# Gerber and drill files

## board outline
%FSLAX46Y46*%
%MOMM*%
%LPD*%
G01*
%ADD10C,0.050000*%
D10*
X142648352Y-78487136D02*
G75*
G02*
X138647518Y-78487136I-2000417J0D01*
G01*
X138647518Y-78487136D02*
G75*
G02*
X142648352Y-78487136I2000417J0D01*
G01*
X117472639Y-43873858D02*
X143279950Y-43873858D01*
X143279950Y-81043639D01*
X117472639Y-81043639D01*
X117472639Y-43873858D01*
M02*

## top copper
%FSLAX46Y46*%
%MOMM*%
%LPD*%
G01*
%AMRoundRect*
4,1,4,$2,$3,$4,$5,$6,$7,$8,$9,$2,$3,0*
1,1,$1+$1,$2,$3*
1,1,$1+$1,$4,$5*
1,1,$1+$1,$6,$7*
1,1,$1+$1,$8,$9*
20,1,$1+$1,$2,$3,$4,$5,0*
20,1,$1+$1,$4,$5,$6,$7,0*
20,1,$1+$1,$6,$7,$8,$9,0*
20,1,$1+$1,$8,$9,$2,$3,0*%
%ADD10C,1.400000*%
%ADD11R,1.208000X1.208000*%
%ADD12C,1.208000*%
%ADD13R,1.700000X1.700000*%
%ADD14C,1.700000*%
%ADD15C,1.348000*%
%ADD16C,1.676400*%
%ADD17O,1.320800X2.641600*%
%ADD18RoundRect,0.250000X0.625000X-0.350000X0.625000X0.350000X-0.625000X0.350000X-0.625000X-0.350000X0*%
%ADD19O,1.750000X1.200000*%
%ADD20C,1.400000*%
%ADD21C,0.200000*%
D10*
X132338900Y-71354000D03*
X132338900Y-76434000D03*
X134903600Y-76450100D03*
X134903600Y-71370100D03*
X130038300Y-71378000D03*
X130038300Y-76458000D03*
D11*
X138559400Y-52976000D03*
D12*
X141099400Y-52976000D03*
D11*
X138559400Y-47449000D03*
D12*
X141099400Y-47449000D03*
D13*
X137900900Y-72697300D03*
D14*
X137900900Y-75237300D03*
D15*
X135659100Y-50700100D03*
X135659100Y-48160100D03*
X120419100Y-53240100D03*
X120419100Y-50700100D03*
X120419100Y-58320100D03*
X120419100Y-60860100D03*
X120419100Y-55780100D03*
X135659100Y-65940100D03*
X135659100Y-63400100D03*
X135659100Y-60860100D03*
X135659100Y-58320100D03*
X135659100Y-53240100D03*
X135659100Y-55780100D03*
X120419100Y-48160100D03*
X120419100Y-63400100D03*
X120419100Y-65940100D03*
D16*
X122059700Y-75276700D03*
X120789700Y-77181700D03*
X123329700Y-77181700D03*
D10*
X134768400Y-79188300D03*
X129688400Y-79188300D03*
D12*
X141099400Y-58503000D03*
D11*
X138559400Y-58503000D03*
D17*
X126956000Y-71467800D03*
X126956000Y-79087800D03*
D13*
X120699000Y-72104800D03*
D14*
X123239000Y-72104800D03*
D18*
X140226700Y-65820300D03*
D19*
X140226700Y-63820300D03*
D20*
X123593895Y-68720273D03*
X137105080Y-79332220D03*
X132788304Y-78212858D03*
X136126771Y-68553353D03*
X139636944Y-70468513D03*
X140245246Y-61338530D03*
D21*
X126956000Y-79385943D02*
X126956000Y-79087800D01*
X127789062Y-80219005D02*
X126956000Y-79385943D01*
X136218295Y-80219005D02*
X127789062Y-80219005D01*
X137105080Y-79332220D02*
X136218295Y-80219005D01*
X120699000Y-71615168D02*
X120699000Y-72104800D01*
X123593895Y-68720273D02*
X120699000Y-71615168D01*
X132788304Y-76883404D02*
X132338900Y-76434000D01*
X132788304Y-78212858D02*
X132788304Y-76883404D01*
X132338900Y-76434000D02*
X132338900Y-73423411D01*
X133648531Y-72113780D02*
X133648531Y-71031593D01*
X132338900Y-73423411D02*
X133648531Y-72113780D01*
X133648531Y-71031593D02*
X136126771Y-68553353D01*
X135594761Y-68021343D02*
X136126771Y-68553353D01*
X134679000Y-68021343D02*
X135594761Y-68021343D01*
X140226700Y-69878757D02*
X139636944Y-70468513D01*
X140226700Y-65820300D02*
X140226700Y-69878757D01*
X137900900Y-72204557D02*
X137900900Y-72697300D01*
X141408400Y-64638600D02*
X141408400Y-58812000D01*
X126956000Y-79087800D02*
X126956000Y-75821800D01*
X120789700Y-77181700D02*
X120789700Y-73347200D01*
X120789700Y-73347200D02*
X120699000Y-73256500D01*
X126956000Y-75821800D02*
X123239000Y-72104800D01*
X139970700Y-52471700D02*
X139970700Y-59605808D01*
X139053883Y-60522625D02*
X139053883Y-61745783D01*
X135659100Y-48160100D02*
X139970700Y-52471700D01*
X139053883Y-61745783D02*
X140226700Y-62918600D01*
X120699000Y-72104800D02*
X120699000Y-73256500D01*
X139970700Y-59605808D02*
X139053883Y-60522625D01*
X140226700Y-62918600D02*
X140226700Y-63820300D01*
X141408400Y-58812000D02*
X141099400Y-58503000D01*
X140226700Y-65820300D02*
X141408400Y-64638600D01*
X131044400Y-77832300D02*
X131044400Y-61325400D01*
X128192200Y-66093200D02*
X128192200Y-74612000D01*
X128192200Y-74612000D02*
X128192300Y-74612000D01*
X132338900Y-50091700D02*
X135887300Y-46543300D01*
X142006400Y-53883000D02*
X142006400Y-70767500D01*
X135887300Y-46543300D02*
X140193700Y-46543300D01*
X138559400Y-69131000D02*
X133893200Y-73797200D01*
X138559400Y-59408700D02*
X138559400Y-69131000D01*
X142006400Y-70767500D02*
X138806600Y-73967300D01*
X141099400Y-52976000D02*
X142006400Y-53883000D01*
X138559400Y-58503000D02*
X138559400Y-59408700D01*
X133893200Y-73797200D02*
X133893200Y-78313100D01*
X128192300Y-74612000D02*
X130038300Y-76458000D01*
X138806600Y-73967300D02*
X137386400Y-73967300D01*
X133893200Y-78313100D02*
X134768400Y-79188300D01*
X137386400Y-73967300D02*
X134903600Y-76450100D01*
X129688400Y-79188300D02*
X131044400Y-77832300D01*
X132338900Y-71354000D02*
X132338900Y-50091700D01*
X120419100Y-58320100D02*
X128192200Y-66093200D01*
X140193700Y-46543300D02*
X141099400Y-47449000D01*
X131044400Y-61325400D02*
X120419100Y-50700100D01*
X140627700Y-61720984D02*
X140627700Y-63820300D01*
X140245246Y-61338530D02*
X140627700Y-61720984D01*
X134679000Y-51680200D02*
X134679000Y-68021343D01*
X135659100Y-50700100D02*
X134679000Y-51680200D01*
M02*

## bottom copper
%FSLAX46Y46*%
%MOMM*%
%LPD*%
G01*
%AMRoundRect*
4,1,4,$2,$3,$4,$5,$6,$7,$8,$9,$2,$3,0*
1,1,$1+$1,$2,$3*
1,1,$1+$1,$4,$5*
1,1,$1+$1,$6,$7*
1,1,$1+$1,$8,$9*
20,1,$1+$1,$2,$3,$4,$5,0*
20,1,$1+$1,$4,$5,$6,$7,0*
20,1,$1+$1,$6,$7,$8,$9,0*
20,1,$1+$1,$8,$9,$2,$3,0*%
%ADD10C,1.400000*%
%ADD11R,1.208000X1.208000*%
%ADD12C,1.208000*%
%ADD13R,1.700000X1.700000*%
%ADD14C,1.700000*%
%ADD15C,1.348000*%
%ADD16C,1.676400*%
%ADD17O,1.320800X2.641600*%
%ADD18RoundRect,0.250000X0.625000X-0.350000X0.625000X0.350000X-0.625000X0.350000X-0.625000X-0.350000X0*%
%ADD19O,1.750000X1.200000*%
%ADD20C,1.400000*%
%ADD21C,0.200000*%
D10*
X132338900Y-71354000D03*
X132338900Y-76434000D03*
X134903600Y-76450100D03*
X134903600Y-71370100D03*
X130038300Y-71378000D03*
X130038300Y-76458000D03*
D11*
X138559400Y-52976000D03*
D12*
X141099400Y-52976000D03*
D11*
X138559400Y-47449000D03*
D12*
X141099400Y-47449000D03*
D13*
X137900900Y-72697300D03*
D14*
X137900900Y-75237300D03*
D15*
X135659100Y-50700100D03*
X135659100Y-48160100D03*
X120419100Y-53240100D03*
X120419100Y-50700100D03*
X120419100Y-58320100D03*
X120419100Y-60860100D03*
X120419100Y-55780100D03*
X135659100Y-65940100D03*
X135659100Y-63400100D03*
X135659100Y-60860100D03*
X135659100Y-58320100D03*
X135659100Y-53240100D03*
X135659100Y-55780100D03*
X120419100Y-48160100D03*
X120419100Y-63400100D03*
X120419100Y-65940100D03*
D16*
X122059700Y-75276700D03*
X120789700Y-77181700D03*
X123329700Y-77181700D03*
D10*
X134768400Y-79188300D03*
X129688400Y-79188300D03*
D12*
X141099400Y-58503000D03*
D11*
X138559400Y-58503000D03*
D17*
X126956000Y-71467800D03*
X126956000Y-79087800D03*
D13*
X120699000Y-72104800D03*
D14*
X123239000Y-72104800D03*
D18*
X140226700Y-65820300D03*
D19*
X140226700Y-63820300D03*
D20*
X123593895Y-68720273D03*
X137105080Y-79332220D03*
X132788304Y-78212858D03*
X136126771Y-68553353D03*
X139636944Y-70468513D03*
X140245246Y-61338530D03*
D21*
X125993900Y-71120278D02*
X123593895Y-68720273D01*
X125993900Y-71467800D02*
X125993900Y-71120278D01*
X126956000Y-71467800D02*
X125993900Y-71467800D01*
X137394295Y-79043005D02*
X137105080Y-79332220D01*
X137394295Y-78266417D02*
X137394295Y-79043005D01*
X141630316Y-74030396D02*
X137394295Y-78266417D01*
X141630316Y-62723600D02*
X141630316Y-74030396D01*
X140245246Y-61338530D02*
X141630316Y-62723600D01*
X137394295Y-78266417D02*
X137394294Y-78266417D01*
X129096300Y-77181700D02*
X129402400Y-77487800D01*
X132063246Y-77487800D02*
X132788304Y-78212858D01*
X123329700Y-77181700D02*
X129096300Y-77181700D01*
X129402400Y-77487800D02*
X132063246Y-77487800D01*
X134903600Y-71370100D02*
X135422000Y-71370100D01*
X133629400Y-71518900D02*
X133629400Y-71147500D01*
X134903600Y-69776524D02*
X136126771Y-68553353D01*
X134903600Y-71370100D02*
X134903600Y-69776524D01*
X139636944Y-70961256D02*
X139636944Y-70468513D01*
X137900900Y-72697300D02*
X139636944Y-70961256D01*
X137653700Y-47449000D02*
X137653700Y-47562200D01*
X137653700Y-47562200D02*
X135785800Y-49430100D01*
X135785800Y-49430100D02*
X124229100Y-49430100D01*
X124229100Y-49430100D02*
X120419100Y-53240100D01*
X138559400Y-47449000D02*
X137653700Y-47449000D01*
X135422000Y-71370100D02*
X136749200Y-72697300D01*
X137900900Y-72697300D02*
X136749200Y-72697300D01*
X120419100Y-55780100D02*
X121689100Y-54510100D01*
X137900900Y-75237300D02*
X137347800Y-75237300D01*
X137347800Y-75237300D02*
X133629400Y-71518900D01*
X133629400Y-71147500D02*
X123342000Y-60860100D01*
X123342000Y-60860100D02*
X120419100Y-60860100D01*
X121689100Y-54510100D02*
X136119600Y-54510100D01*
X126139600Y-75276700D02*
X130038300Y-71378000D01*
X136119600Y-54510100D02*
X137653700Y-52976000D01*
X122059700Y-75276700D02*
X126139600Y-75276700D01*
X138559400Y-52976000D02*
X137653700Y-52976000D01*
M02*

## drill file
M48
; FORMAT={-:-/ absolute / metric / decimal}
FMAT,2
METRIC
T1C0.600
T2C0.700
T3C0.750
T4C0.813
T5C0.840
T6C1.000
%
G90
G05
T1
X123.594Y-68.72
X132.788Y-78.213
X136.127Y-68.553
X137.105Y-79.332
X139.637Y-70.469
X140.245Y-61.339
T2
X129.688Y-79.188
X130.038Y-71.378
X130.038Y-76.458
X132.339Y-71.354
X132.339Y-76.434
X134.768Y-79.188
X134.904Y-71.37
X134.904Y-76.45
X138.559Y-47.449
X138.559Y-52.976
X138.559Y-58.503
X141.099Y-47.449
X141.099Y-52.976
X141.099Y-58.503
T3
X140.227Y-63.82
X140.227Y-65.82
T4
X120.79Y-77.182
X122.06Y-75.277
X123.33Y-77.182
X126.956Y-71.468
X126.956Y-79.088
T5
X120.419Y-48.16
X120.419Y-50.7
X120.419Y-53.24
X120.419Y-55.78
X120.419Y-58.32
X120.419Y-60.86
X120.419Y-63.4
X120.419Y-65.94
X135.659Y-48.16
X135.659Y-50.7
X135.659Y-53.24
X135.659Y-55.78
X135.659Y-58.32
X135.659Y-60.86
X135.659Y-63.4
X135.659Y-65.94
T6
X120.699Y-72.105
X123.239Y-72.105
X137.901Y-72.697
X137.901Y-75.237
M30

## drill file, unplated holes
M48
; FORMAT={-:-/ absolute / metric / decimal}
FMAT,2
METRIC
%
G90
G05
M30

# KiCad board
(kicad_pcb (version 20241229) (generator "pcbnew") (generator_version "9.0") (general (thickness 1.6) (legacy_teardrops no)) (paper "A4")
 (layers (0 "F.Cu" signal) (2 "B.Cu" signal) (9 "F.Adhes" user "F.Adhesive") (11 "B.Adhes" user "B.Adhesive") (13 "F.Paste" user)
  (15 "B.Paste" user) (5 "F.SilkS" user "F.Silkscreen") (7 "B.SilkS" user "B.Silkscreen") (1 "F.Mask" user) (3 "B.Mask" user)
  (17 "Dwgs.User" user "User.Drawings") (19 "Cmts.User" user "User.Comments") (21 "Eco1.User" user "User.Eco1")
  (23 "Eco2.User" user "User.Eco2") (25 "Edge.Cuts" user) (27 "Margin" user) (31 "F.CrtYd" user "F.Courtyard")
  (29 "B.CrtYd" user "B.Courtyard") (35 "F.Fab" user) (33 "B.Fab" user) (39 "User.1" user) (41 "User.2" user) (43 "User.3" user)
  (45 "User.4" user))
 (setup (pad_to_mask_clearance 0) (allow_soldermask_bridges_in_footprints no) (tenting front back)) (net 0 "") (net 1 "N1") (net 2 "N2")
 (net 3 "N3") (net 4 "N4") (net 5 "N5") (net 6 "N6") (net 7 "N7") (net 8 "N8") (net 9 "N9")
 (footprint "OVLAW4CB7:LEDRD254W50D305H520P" (layer "F.Cu") (at 139.8294 52.976)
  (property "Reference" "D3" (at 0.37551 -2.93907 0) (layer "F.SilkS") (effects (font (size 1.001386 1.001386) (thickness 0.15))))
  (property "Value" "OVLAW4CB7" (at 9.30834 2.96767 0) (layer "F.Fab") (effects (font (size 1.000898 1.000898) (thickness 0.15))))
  (pad "A" thru_hole rect (at -1.27 0) (size 1.208 1.208) (drill 0.7) (layers "*.Cu" "*.Mask") (remove_unused_layers no)
   (solder_mask_margin 0.102))
  (pad "C" thru_hole circle (at 1.27 0) (size 1.208 1.208) (drill 0.7) (layers "*.Cu" "*.Mask") (remove_unused_layers no)
   (solder_mask_margin 0.102)))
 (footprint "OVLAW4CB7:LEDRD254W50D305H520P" (layer "F.Cu") (at 139.8294 47.449)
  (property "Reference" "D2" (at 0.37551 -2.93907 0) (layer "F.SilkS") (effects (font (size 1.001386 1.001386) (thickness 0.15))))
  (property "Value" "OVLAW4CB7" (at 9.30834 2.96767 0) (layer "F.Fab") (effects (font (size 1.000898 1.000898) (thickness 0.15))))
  (pad "A" thru_hole rect (at -1.27 0) (size 1.208 1.208) (drill 0.7) (layers "*.Cu" "*.Mask") (remove_unused_layers no)
   (solder_mask_margin 0.102))
  (pad "C" thru_hole circle (at 1.27 0) (size 1.208 1.208) (drill 0.7) (layers "*.Cu" "*.Mask") (remove_unused_layers no)
   (solder_mask_margin 0.102)))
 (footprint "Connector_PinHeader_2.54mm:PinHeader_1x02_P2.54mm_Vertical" (layer "F.Cu") (at 137.9009 72.6973)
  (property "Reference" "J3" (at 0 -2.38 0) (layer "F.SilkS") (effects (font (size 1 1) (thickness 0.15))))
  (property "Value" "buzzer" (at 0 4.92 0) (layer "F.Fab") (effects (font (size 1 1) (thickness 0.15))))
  (pad "1" thru_hole rect (at 0 0) (size 1.7 1.7) (drill 1) (layers "*.Cu" "*.Mask") (remove_unused_layers no))
  (pad "2" thru_hole circle (at 0 2.54) (size 1.7 1.7) (drill 1) (layers "*.Cu" "*.Mask") (remove_unused_layers no)))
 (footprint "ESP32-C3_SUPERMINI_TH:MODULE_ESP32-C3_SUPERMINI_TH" (layer "F.Cu") (at 128.0391 58.0601)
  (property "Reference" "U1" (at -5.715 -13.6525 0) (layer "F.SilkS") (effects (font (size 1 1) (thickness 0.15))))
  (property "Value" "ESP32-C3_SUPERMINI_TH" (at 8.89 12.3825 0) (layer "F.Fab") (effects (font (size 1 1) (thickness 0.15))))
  (pad "0" thru_hole circle (at 7.62 7.88) (size 1.348 1.348) (drill 0.84) (layers "*.Cu" "*.Mask") (remove_unused_layers no) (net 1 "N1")
   (solder_mask_margin 0.102))
  (pad "1" thru_hole circle (at 7.62 5.34) (size 1.348 1.348) (drill 0.84) (layers "*.Cu" "*.Mask") (remove_unused_layers no) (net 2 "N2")
   (solder_mask_margin 0.102))
  (pad "2" thru_hole circle (at 7.62 2.8) (size 1.348 1.348) (drill 0.84) (layers "*.Cu" "*.Mask") (remove_unused_layers no) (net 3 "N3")
   (solder_mask_margin 0.102))
  (pad "3" thru_hole circle (at 7.62 0.26) (size 1.348 1.348) (drill 0.84) (layers "*.Cu" "*.Mask") (remove_unused_layers no) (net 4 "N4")
   (solder_mask_margin 0.102))
  (pad "3.3" thru_hole circle (at 7.62 -4.82) (size 1.348 1.348) (drill 0.84) (layers "*.Cu" "*.Mask") (remove_unused_layers no)
   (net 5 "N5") (solder_mask_margin 0.102))
  (pad "4" thru_hole circle (at 7.62 -2.28) (size 1.348 1.348) (drill 0.84) (layers "*.Cu" "*.Mask") (remove_unused_layers no) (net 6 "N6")
   (solder_mask_margin 0.102))
  (pad "5" thru_hole circle (at -7.62 -9.9) (size 1.348 1.348) (drill 0.84) (layers "*.Cu" "*.Mask") (remove_unused_layers no) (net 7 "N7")
   (solder_mask_margin 0.102))
  (pad "5V" thru_hole circle (at 7.62 -9.9) (size 1.348 1.348) (drill 0.84) (layers "*.Cu" "*.Mask") (remove_unused_layers no)
   (solder_mask_margin 0.102))
  (pad "6" thru_hole circle (at -7.62 -7.36) (size 1.348 1.348) (drill 0.84) (layers "*.Cu" "*.Mask") (remove_unused_layers no)
   (solder_mask_margin 0.102))
  (pad "7" thru_hole circle (at -7.62 -4.82) (size 1.348 1.348) (drill 0.84) (layers "*.Cu" "*.Mask") (remove_unused_layers no)
   (solder_mask_margin 0.102))
  (pad "8" thru_hole circle (at -7.62 -2.28) (size 1.348 1.348) (drill 0.84) (layers "*.Cu" "*.Mask") (remove_unused_layers no)
   (solder_mask_margin 0.102))
  (pad "9" thru_hole circle (at -7.62 0.26) (size 1.348 1.348) (drill 0.84) (layers "*.Cu" "*.Mask") (remove_unused_layers no)
   (solder_mask_margin 0.102))
  (pad "10" thru_hole circle (at -7.62 2.8) (size 1.348 1.348) (drill 0.84) (layers "*.Cu" "*.Mask") (remove_unused_layers no)
   (solder_mask_margin 0.102))
  (pad "20" thru_hole circle (at -7.62 5.34) (size 1.348 1.348) (drill 0.84) (layers "*.Cu" "*.Mask") (remove_unused_layers no) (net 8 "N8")
   (solder_mask_margin 0.102))
  (pad "21" thru_hole circle (at -7.62 7.88) (size 1.348 1.348) (drill 0.84) (layers "*.Cu" "*.Mask") (remove_unused_layers no) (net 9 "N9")
   (solder_mask_margin 0.102))
  (pad "G" thru_hole circle (at 7.62 -7.36) (size 1.348 1.348) (drill 0.84) (layers "*.Cu" "*.Mask") (remove_unused_layers no)
   (solder_mask_margin 0.102)))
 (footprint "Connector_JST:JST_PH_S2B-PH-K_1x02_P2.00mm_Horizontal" (layer "F.Cu") (at 140.2267 65.8203 90)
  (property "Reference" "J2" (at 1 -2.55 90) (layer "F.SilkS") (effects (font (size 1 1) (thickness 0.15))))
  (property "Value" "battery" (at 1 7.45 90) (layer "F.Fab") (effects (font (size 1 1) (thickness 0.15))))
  (pad "1" thru_hole roundrect (at 0 0 90) (size 1.2 1.75) (drill 0.75) (layers "*.Cu" "*.Mask") (remove_unused_layers no)
   (roundrect_rratio 0.208333))
  (pad "2" thru_hole oval (at 2 0 90) (size 1.2 1.75) (drill 0.75) (layers "*.Cu" "*.Mask") (remove_unused_layers no)))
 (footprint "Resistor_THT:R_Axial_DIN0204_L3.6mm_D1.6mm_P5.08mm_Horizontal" (layer "F.Cu") (at 134.9036 76.4501 90)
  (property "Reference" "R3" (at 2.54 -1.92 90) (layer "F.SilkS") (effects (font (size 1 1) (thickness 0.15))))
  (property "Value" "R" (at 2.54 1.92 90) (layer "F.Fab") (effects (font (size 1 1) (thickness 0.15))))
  (pad "1" thru_hole circle (at 0 0 90) (size 1.4 1.4) (drill 0.7) (layers "*.Cu" "*.Mask") (remove_unused_layers no))
  (pad "2" thru_hole circle (at 5.08 0 90) (size 1.4 1.4) (drill 0.7) (layers "*.Cu" "*.Mask") (remove_unused_layers no)))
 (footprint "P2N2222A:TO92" (layer "F.Cu") (at 122.0597 77.1817)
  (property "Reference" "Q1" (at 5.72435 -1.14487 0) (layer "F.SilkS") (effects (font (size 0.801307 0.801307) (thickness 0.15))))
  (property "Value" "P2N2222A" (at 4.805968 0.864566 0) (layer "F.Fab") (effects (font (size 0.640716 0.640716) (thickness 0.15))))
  (pad "1" thru_hole circle (at 1.27 0) (size 1.6764 1.6764) (drill 0.8128) (layers "*.Cu" "*.Mask") (remove_unused_layers no)
   (solder_mask_margin 0.102))
  (pad "2" thru_hole circle (at 0 -1.905) (size 1.6764 1.6764) (drill 0.8128) (layers "*.Cu" "*.Mask") (remove_unused_layers no)
   (solder_mask_margin 0.102))
  (pad "3" thru_hole circle (at -1.27 0) (size 1.6764 1.6764) (drill 0.8128) (layers "*.Cu" "*.Mask") (remove_unused_layers no)
   (solder_mask_margin 0.102)))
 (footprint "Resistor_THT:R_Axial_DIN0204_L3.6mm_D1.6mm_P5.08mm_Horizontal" (layer "F.Cu") (at 130.0383 76.458 90)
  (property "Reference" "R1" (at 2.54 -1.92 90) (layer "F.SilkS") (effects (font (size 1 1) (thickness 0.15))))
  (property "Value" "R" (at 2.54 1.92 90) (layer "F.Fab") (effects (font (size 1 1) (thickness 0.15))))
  (pad "1" thru_hole circle (at 0 0 90) (size 1.4 1.4) (drill 0.7) (layers "*.Cu" "*.Mask") (remove_unused_layers no))
  (pad "2" thru_hole circle (at 5.08 0 90) (size 1.4 1.4) (drill 0.7) (layers "*.Cu" "*.Mask") (remove_unused_layers no)))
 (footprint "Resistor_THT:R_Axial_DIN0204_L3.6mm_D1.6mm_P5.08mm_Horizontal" (layer "F.Cu") (at 132.3389 71.354 -90)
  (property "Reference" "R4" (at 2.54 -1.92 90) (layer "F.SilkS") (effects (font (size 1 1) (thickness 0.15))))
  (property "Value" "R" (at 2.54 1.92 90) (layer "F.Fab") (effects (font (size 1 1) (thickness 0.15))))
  (pad "1" thru_hole circle (at 0 0 270) (size 1.4 1.4) (drill 0.7) (layers "*.Cu" "*.Mask") (remove_unused_layers no))
  (pad "2" thru_hole circle (at 5.08 0 270) (size 1.4 1.4) (drill 0.7) (layers "*.Cu" "*.Mask") (remove_unused_layers no)))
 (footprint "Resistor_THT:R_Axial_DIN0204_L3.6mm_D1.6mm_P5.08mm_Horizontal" (layer "F.Cu") (at 134.7684 79.1883 180)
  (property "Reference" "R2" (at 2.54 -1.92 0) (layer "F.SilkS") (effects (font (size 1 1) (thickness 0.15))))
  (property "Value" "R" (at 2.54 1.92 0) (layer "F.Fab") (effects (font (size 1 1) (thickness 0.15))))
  (pad "1" thru_hole circle (at 0 0 180) (size 1.4 1.4) (drill 0.7) (layers "*.Cu" "*.Mask") (remove_unused_layers no))
  (pad "2" thru_hole circle (at 5.08 0 180) (size 1.4 1.4) (drill 0.7) (layers "*.Cu" "*.Mask") (remove_unused_layers no)))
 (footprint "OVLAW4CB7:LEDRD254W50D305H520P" (layer "F.Cu") (at 139.8294 58.503)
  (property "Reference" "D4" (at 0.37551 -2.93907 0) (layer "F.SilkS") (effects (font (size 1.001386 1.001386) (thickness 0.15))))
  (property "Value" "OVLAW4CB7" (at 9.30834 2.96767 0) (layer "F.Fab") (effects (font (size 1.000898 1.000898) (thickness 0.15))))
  (pad "A" thru_hole rect (at -1.27 0) (size 1.208 1.208) (drill 0.7) (layers "*.Cu" "*.Mask") (remove_unused_layers no)
   (solder_mask_margin 0.102))
  (pad "C" thru_hole circle (at 1.27 0) (size 1.208 1.208) (drill 0.7) (layers "*.Cu" "*.Mask") (remove_unused_layers no)
   (solder_mask_margin 0.102)))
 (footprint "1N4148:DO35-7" (layer "F.Cu") (at 126.956 75.2778 90)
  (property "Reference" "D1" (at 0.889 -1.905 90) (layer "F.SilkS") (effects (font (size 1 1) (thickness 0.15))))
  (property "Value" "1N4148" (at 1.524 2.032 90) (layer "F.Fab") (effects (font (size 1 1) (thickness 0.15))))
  (pad "A" thru_hole oval (at 3.81 0 90) (size 2.6416 1.3208) (drill 0.8128) (layers "*.Cu" "*.Mask") (remove_unused_layers no)
   (solder_mask_margin 0.102))
  (pad "C" thru_hole oval (at -3.81 0 90) (size 2.6416 1.3208) (drill 0.8128) (layers "*.Cu" "*.Mask") (remove_unused_layers no)
   (solder_mask_margin 0.102)))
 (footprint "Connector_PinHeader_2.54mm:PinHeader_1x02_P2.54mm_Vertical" (layer "F.Cu") (at 120.699 72.1048 90)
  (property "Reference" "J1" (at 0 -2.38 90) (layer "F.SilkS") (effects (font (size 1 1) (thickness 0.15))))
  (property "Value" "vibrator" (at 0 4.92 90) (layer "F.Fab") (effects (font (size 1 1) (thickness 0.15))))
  (pad "1" thru_hole rect (at 0 0 90) (size 1.7 1.7) (drill 1) (layers "*.Cu" "*.Mask") (remove_unused_layers no))
  (pad "2" thru_hole circle (at 0 2.54 90) (size 1.7 1.7) (drill 1) (layers "*.Cu" "*.Mask") (remove_unused_layers no)))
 (gr_circle (center 140.647935 78.487136) (end 138.891232 79.444039) (stroke (width 0.05) (type default)) (fill no) (layer "Edge.Cuts"))
 (gr_rect (start 117.472639 43.873858) (end 143.27995 81.043639) (stroke (width 0.05) (type default)) (fill no) (layer "Edge.Cuts"))
 (segment (start 127.789062 80.219005) (end 126.956 79.385943) (width 0.2) (layer "F.Cu") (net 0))
 (segment (start 132.788304 78.212858) (end 132.788304 76.883404) (width 0.2) (layer "F.Cu") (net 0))
 (segment (start 137.3864 73.9673) (end 134.9036 76.4501) (width 0.2) (layer "F.Cu") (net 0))
 (segment (start 140.1937 46.5433) (end 141.0994 47.449) (width 0.2) (layer "F.Cu") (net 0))
 (segment (start 128.1923 74.612) (end 130.0383 76.458) (width 0.2) (layer "F.Cu") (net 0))
 (segment (start 138.8066 73.9673) (end 137.3864 73.9673) (width 0.2) (layer "F.Cu") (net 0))
 (segment (start 134.679 51.6802) (end 134.679 68.021343) (width 0.2) (layer "F.Cu") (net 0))
 (segment (start 140.2267 65.8203) (end 140.2267 69.878757) (width 0.2) (layer "F.Cu") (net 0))
 (segment (start 120.7897 77.1817) (end 120.7897 73.3472) (width 0.2) (layer "F.Cu") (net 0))
 (segment (start 139.9707 52.4717) (end 139.9707 59.605808) (width 0.2) (layer "F.Cu") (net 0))
 (segment (start 136.218295 80.219005) (end 127.789062 80.219005) (width 0.2) (layer "F.Cu") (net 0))
 (segment (start 141.4084 58.812) (end 141.0994 58.503) (width 0.2) (layer "F.Cu") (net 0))
 (segment (start 132.3389 71.354) (end 132.3389 50.0917) (width 0.2) (layer "F.Cu") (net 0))
 (segment (start 142.0064 70.7675) (end 138.8066 73.9673) (width 0.2) (layer "F.Cu") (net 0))
 (segment (start 132.3389 50.0917) (end 135.8873 46.5433) (width 0.2) (layer "F.Cu") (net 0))
 (segment (start 133.648531 72.11378) (end 133.648531 71.031593) (width 0.2) (layer "F.Cu") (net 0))
 (segment (start 120.699 72.1048) (end 120.699 73.2565) (width 0.2) (layer "F.Cu") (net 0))
 (segment (start 135.594761 68.021343) (end 136.126771 68.553353) (width 0.2) (layer "F.Cu") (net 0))
 (segment (start 133.8932 78.3131) (end 134.7684 79.1883) (width 0.2) (layer "F.Cu") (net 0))
 (segment (start 140.2267 62.9186) (end 140.2267 63.8203) (width 0.2) (layer "F.Cu") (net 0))
 (segment (start 135.6591 50.7001) (end 134.679 51.6802) (width 0.2) (layer "F.Cu") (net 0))
 (segment (start 140.2267 65.8203) (end 141.4084 64.6386) (width 0.2) (layer "F.Cu") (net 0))
 (segment (start 131.0444 61.3254) (end 120.4191 50.7001) (width 0.2) (layer "F.Cu") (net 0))
 (segment (start 132.3389 76.434) (end 132.3389 73.423411) (width 0.2) (layer "F.Cu") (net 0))
 (segment (start 126.956 79.385943) (end 126.956 79.0878) (width 0.2) (layer "F.Cu") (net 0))
 (segment (start 123.593895 68.720273) (end 120.699 71.615168) (width 0.2) (layer "F.Cu") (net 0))
 (segment (start 134.679 68.021343) (end 135.594761 68.021343) (width 0.2) (layer "F.Cu") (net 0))
 (segment (start 120.4191 58.3201) (end 128.1922 66.0932) (width 0.2) (layer "F.Cu") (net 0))
 (segment (start 126.956 79.0878) (end 126.956 75.8218) (width 0.2) (layer "F.Cu") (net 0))
 (segment (start 135.6591 48.1601) (end 139.9707 52.4717) (width 0.2) (layer "F.Cu") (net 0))
 (segment (start 140.6277 61.720984) (end 140.6277 63.8203) (width 0.2) (layer "F.Cu") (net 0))
 (segment (start 128.1922 66.0932) (end 128.1922 74.612) (width 0.2) (layer "F.Cu") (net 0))
 (segment (start 126.956 75.8218) (end 123.239 72.1048) (width 0.2) (layer "F.Cu") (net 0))
 (segment (start 128.1922 74.612) (end 128.1923 74.612) (width 0.2) (layer "F.Cu") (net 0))
 (segment (start 139.9707 59.605808) (end 139.053883 60.522625) (width 0.2) (layer "F.Cu") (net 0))
 (segment (start 133.648531 71.031593) (end 136.126771 68.553353) (width 0.2) (layer "F.Cu") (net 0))
 (segment (start 142.0064 53.883) (end 142.0064 70.7675) (width 0.2) (layer "F.Cu") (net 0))
 (segment (start 135.8873 46.5433) (end 140.1937 46.5433) (width 0.2) (layer "F.Cu") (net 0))
 (segment (start 140.2267 69.878757) (end 139.636944 70.468513) (width 0.2) (layer "F.Cu") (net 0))
 (segment (start 131.0444 77.8323) (end 131.0444 61.3254) (width 0.2) (layer "F.Cu") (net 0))
 (segment (start 140.245246 61.33853) (end 140.6277 61.720984) (width 0.2) (layer "F.Cu") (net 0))
 (segment (start 141.4084 64.6386) (end 141.4084 58.812) (width 0.2) (layer "F.Cu") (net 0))
 (segment (start 137.9009 72.204557) (end 137.9009 72.6973) (width 0.2) (layer "F.Cu") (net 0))
 (segment (start 129.6884 79.1883) (end 131.0444 77.8323) (width 0.2) (layer "F.Cu") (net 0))
 (segment (start 138.5594 58.503) (end 138.5594 59.4087) (width 0.2) (layer "F.Cu") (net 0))
 (segment (start 132.3389 73.423411) (end 133.648531 72.11378) (width 0.2) (layer "F.Cu") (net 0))
 (segment (start 132.788304 76.883404) (end 132.3389 76.434) (width 0.2) (layer "F.Cu") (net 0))
 (segment (start 139.053883 61.745783) (end 140.2267 62.9186) (width 0.2) (layer "F.Cu") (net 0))
 (segment (start 141.0994 52.976) (end 142.0064 53.883) (width 0.2) (layer "F.Cu") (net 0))
 (segment (start 139.053883 60.522625) (end 139.053883 61.745783) (width 0.2) (layer "F.Cu") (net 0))
 (segment (start 120.699 71.615168) (end 120.699 72.1048) (width 0.2) (layer "F.Cu") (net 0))
 (segment (start 138.5594 69.131) (end 133.8932 73.7972) (width 0.2) (layer "F.Cu") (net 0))
 (segment (start 120.7897 73.3472) (end 120.699 73.2565) (width 0.2) (layer "F.Cu") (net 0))
 (segment (start 133.8932 73.7972) (end 133.8932 78.3131) (width 0.2) (layer "F.Cu") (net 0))
 (segment (start 137.10508 79.33222) (end 136.218295 80.219005) (width 0.2) (layer "F.Cu") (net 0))
 (segment (start 138.5594 59.4087) (end 138.5594 69.131) (width 0.2) (layer "F.Cu") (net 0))
 (via (at 123.593895 68.720273) (size 1.4) (drill 0.6) (layers "F.Cu" "B.Cu") (free yes) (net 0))
 (via (at 140.245246 61.33853) (size 1.4) (drill 0.6) (layers "F.Cu" "B.Cu") (free yes) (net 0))
 (via (at 139.636944 70.468513) (size 1.4) (drill 0.6) (layers "F.Cu" "B.Cu") (free yes) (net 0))
 (via (at 136.126771 68.553353) (size 1.4) (drill 0.6) (layers "F.Cu" "B.Cu") (free yes) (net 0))
 (via (at 132.788304 78.212858) (size 1.4) (drill 0.6) (layers "F.Cu" "B.Cu") (free yes) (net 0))
 (via (at 137.10508 79.33222) (size 1.4) (drill 0.6) (layers "F.Cu" "B.Cu") (free yes) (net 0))
 (segment (start 141.630316 74.030396) (end 137.394295 78.266417) (width 0.2) (layer "B.Cu") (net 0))
 (segment (start 125.9939 71.120278) (end 123.593895 68.720273) (width 0.2) (layer "B.Cu") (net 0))
 (segment (start 137.9009 72.6973) (end 139.636944 70.961256) (width 0.2) (layer "B.Cu") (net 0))
 (segment (start 140.245246 61.33853) (end 141.630316 62.7236) (width 0.2) (layer "B.Cu") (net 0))
 (segment (start 134.9036 71.3701) (end 134.9036 69.776524) (width 0.2) (layer "B.Cu") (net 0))
 (segment (start 129.0963 77.1817) (end 129.4024 77.4878) (width 0.2) (layer "B.Cu") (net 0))
 (segment (start 126.1396 75.2767) (end 130.0383 71.378) (width 0.2) (layer "B.Cu") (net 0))
 (segment (start 138.5594 52.976) (end 137.6537 52.976) (width 0.2) (layer "B.Cu") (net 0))
 (segment (start 123.342 60.8601) (end 120.4191 60.8601) (width 0.2) (layer "B.Cu") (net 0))
 (segment (start 137.6537 47.449) (end 137.6537 47.5622) (width 0.2) (layer "B.Cu") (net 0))
 (segment (start 137.6537 47.5622) (end 135.7858 49.4301) (width 0.2) (layer "B.Cu") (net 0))
 (segment (start 135.7858 49.4301) (end 124.2291 49.4301) (width 0.2) (layer "B.Cu") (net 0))
 (segment (start 137.3478 75.2373) (end 133.6294 71.5189) (width 0.2) (layer "B.Cu") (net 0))
 (segment (start 138.5594 47.449) (end 137.6537 47.449) (width 0.2) (layer "B.Cu") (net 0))
 (segment (start 120.4191 55.7801) (end 121.6891 54.5101) (width 0.2) (layer "B.Cu") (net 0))
 (segment (start 135.422 71.3701) (end 136.7492 72.6973) (width 0.2) (layer "B.Cu") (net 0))
 (segment (start 133.6294 71.5189) (end 133.6294 71.1475) (width 0.2) (layer "B.Cu") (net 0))
 (segment (start 137.9009 75.2373) (end 137.3478 75.2373) (width 0.2) (layer "B.Cu") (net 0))
 (segment (start 137.394295 78.266417) (end 137.394294 78.266417) (width 0.2) (layer "B.Cu") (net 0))
 (segment (start 134.9036 69.776524) (end 136.126771 68.553353) (width 0.2) (layer "B.Cu") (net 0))
 (segment (start 126.956 71.4678) (end 125.9939 71.4678) (width 0.2) (layer "B.Cu") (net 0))
 (segment (start 125.9939 71.4678) (end 125.9939 71.120278) (width 0.2) (layer "B.Cu") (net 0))
 (segment (start 129.4024 77.4878) (end 132.063246 77.4878) (width 0.2) (layer "B.Cu") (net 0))
 (segment (start 137.9009 72.6973) (end 136.7492 72.6973) (width 0.2) (layer "B.Cu") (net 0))
 (segment (start 134.9036 71.3701) (end 135.422 71.3701) (width 0.2) (layer "B.Cu") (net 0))
 (segment (start 137.394295 78.266417) (end 137.394295 79.043005) (width 0.2) (layer "B.Cu") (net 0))
 (segment (start 132.063246 77.4878) (end 132.788304 78.212858) (width 0.2) (layer "B.Cu") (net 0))
 (segment (start 121.6891 54.5101) (end 136.1196 54.5101) (width 0.2) (layer "B.Cu") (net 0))
 (segment (start 137.394295 79.043005) (end 137.10508 79.33222) (width 0.2) (layer "B.Cu") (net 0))
 (segment (start 141.630316 62.7236) (end 141.630316 74.030396) (width 0.2) (layer "B.Cu") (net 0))
 (segment (start 136.1196 54.5101) (end 137.6537 52.976) (width 0.2) (layer "B.Cu") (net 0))
 (segment (start 124.2291 49.4301) (end 120.4191 53.2401) (width 0.2) (layer "B.Cu") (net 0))
 (segment (start 139.636944 70.961256) (end 139.636944 70.468513) (width 0.2) (layer "B.Cu") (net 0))
 (segment (start 133.6294 71.1475) (end 123.342 60.8601) (width 0.2) (layer "B.Cu") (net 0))
 (segment (start 122.0597 75.2767) (end 126.1396 75.2767) (width 0.2) (layer "B.Cu") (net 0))
 (segment (start 123.3297 77.1817) (end 129.0963 77.1817) (width 0.2) (layer "B.Cu") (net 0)))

